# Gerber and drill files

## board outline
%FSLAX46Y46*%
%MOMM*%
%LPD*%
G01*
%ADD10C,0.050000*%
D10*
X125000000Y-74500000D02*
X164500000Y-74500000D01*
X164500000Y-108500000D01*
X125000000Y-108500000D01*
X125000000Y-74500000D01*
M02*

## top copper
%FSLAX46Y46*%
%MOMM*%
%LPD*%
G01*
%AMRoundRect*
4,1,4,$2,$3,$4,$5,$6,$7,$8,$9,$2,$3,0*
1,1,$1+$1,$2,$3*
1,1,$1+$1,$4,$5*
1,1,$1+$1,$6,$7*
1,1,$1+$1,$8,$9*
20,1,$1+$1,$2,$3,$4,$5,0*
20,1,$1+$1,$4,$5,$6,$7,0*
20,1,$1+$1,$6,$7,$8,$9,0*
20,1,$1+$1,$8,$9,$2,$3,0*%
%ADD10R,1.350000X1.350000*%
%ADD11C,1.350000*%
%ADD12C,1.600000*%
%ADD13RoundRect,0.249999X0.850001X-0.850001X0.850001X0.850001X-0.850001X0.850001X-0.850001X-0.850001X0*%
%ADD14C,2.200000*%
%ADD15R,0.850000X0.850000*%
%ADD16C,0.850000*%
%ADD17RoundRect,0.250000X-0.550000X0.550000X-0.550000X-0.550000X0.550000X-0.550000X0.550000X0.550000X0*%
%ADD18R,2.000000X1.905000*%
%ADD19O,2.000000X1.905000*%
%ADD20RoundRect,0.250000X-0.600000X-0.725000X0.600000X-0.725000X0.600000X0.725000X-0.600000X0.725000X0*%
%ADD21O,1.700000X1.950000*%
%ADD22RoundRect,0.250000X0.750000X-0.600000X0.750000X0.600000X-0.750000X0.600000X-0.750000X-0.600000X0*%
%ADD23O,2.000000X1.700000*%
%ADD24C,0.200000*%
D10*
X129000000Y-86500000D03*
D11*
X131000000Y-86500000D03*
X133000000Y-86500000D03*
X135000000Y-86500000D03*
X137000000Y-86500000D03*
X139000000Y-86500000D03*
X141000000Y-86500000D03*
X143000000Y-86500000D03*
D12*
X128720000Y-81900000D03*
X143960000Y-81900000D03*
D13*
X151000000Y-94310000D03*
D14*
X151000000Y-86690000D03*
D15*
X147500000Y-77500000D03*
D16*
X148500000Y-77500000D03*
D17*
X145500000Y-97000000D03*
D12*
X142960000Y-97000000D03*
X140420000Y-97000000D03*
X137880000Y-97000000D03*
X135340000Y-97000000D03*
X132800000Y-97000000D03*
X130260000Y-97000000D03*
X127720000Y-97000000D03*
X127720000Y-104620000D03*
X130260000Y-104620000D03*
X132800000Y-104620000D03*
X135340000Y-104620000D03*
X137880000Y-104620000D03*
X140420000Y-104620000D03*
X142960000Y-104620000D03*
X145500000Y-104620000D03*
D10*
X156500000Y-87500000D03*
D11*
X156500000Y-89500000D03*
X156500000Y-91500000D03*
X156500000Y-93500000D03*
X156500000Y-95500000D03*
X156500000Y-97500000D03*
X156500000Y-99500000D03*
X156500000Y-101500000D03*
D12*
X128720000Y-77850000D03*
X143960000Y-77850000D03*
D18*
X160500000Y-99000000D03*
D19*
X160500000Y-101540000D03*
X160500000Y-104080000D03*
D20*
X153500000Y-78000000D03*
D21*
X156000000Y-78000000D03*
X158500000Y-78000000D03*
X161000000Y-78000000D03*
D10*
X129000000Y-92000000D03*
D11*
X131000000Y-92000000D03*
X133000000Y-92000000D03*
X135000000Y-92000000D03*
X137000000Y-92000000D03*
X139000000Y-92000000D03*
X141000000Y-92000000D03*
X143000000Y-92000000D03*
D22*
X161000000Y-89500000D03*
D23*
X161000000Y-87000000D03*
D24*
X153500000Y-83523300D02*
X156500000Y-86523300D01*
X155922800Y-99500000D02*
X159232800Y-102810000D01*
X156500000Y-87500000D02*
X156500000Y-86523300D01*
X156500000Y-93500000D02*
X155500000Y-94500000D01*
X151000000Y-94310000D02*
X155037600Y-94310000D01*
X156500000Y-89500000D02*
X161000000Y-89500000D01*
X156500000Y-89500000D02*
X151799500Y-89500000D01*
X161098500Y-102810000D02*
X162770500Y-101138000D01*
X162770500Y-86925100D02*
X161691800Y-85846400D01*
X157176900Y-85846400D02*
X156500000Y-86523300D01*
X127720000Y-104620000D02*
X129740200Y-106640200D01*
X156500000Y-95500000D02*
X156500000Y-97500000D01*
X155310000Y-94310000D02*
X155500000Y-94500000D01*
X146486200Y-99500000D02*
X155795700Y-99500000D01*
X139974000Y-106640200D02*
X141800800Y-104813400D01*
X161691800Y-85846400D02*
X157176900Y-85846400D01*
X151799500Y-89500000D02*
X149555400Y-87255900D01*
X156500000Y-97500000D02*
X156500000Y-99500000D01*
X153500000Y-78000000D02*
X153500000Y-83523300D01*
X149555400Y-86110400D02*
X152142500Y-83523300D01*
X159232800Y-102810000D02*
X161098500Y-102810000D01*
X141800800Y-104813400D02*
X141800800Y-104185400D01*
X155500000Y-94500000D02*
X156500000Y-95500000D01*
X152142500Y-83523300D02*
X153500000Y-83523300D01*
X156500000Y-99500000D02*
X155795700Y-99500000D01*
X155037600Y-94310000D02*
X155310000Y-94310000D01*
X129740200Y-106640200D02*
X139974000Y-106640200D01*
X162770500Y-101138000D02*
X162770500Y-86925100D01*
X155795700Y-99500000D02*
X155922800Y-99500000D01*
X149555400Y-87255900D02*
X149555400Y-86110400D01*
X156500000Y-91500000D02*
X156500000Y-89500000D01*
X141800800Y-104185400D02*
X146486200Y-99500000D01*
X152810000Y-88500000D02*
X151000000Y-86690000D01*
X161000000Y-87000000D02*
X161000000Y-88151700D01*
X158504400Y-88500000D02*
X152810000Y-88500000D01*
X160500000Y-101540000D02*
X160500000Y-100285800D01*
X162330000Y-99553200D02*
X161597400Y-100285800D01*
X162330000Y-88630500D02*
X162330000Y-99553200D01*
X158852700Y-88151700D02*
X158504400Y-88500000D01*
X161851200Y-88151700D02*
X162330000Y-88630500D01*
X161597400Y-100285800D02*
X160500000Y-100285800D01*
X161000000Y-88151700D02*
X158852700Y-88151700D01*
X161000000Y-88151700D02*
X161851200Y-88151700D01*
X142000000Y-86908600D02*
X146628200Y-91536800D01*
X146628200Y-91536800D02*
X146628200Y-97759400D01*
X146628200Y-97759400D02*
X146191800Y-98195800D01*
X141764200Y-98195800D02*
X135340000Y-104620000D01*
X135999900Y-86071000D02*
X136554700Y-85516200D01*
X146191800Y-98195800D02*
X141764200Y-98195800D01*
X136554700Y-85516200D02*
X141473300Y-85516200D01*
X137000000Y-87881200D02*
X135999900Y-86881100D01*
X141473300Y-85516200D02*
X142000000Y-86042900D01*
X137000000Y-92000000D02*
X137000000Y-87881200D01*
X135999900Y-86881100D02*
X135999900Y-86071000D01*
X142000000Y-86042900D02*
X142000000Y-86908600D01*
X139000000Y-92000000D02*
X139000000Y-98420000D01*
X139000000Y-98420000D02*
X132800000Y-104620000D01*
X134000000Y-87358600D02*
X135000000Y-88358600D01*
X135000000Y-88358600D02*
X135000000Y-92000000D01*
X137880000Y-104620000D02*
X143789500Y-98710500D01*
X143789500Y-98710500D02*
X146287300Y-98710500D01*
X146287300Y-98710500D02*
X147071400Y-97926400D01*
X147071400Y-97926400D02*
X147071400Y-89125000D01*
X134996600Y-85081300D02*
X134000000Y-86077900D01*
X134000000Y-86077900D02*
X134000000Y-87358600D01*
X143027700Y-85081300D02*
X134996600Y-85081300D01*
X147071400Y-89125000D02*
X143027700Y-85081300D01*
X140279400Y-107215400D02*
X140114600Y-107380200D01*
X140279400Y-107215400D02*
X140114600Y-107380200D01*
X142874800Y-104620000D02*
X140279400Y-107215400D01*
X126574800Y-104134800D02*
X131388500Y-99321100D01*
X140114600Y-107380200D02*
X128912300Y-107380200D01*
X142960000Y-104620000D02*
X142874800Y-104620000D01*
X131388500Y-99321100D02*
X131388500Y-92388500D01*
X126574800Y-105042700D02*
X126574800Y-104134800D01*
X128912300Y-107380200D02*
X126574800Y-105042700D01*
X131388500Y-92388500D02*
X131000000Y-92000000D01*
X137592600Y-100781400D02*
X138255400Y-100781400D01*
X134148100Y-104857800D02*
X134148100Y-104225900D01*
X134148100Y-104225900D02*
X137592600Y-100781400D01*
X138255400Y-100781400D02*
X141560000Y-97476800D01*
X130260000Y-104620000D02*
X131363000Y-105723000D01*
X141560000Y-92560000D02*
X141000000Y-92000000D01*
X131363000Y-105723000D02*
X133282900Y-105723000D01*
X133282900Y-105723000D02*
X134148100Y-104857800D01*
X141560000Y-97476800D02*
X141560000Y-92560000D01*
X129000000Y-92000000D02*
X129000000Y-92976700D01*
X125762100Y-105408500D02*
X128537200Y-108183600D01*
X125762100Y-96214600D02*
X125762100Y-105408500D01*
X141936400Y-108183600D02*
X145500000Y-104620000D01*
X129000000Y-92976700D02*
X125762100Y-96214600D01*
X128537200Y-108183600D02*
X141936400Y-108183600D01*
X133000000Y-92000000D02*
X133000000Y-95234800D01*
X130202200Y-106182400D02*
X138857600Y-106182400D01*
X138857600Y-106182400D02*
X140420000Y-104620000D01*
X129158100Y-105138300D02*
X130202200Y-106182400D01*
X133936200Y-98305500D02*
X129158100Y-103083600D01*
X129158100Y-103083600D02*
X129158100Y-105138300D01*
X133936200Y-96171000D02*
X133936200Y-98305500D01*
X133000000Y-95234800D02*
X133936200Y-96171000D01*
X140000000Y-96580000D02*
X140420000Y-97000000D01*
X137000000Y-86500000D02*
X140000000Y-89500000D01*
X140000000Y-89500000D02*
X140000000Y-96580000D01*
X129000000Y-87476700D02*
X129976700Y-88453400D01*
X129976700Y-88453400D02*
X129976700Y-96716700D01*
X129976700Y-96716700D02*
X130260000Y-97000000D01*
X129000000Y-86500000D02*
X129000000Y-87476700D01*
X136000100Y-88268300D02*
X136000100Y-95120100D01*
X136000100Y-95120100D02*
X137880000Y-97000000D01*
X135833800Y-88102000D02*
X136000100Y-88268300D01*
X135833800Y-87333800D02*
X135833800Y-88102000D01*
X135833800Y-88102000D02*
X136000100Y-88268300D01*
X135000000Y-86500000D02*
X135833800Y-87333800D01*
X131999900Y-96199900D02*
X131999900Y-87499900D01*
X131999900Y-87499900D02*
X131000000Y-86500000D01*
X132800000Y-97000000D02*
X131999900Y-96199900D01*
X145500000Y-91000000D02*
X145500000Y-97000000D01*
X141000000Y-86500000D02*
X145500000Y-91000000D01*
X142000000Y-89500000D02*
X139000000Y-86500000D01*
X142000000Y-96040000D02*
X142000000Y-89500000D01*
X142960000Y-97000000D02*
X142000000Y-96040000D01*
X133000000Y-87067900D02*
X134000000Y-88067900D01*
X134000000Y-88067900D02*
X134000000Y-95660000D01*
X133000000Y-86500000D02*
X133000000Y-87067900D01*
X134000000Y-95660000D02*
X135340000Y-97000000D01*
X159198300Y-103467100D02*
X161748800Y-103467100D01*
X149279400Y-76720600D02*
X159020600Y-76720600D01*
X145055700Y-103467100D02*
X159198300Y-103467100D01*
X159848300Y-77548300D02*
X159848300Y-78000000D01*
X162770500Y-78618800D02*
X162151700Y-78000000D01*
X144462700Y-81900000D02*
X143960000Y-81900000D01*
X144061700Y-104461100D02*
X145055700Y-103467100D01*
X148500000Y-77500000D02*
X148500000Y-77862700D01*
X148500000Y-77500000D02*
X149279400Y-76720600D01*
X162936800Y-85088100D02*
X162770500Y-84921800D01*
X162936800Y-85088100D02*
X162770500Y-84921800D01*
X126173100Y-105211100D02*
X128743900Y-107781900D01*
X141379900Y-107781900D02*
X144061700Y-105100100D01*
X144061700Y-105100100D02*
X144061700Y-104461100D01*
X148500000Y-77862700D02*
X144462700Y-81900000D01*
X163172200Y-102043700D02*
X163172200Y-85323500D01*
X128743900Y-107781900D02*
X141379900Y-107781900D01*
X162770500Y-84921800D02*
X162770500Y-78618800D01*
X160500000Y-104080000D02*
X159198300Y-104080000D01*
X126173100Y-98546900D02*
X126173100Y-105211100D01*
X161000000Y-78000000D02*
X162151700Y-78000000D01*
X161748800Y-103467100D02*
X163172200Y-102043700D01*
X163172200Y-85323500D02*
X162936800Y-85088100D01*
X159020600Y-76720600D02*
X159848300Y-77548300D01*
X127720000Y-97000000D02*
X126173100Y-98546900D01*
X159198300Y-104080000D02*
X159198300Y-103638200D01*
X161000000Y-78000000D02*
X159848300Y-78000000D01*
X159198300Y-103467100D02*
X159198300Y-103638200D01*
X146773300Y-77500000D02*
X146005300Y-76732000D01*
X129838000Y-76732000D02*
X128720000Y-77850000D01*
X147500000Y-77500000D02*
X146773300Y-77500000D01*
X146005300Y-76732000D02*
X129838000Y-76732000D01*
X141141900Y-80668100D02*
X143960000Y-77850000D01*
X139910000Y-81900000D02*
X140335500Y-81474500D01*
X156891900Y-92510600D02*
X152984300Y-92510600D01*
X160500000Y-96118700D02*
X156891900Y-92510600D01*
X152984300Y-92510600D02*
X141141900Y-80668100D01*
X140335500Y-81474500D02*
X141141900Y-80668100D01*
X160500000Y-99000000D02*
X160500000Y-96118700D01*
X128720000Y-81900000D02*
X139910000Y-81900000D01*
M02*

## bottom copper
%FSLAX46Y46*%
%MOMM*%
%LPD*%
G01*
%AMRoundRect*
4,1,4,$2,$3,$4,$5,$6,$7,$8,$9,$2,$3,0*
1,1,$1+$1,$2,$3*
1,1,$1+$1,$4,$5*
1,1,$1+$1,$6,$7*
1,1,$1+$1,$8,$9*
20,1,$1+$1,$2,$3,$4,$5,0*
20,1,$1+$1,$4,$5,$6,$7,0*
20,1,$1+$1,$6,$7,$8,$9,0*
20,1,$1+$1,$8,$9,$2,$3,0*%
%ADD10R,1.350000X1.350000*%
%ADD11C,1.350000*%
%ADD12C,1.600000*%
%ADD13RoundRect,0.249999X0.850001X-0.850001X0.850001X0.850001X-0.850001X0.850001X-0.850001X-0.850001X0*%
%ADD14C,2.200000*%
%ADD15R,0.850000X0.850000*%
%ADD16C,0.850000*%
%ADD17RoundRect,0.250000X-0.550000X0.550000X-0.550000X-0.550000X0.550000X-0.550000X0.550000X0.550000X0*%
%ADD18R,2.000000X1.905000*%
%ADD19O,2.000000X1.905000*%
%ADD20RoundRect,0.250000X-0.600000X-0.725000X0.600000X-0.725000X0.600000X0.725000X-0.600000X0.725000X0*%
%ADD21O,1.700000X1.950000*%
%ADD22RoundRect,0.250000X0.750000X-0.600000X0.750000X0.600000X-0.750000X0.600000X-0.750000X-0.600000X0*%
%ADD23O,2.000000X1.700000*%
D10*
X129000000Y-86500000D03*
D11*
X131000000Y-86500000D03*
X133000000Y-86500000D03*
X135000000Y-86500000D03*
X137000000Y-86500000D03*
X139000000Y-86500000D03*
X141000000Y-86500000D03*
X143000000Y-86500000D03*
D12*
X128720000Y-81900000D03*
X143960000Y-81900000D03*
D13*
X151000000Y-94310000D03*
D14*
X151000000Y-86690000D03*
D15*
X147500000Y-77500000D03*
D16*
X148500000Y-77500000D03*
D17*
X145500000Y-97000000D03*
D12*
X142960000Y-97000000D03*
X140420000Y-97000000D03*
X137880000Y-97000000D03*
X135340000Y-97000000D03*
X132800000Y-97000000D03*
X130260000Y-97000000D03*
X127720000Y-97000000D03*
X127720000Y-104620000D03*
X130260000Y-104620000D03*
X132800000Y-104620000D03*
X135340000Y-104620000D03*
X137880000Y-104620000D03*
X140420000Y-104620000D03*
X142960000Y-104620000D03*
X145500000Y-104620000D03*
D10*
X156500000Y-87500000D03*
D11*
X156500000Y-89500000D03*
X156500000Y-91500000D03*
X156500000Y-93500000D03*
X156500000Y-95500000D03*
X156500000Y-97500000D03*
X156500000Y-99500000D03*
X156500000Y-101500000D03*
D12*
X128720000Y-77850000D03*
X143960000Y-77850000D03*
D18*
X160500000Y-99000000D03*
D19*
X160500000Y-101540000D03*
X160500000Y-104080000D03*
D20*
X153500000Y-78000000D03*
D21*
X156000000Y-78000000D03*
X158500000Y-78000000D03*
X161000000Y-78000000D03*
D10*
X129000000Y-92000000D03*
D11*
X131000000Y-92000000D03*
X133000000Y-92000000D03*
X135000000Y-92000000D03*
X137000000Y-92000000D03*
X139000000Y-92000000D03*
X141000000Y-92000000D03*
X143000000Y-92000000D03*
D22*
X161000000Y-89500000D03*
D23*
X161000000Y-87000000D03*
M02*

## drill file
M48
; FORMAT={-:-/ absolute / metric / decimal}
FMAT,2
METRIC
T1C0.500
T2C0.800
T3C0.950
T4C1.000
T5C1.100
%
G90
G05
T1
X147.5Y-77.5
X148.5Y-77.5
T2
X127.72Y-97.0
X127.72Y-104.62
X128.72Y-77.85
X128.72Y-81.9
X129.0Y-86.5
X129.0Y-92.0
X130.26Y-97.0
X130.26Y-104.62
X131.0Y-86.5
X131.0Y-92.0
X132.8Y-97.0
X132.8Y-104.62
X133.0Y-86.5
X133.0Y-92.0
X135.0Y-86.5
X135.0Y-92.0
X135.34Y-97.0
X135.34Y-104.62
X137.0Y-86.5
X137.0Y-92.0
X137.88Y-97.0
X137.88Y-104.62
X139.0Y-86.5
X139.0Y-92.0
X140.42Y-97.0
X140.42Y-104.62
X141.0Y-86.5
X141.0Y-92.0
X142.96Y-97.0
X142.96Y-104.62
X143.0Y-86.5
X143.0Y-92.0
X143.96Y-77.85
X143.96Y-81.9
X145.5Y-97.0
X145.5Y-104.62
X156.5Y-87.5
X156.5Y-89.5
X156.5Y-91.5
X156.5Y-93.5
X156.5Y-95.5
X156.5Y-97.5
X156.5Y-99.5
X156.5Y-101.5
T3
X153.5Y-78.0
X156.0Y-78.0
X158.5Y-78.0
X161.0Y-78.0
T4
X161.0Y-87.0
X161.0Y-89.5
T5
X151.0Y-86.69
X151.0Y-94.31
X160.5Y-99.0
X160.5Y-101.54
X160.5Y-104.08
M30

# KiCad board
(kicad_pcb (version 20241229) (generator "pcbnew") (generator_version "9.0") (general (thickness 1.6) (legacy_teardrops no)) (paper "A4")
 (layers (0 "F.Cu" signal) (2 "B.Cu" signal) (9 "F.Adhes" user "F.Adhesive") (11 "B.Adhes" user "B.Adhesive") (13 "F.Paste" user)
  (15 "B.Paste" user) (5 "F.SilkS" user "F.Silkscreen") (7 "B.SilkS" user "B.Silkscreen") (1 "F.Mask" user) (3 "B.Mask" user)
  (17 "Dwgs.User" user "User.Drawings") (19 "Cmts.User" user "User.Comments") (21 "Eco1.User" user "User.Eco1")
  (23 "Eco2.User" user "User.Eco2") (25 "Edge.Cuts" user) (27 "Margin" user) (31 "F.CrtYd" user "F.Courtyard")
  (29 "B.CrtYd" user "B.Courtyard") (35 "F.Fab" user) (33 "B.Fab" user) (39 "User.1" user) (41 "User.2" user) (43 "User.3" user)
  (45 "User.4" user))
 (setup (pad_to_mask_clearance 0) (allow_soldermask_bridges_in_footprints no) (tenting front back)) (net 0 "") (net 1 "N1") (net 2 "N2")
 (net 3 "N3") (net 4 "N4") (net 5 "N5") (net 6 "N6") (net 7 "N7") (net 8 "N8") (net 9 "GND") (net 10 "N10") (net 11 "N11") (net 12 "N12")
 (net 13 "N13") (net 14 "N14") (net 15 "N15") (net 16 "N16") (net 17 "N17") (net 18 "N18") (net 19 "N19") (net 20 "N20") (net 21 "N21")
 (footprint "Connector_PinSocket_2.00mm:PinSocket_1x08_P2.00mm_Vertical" (layer "F.Cu") (at 129 86.5 90)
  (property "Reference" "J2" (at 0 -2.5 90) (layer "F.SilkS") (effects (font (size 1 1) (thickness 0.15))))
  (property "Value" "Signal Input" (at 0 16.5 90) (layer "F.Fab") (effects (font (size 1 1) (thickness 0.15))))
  (pad "1" thru_hole rect (at 0 0 90) (size 1.35 1.35) (drill 0.8) (layers "*.Cu" "*.Mask") (remove_unused_layers no) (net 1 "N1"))
  (pad "2" thru_hole circle (at 0 2 90) (size 1.35 1.35) (drill 0.8) (layers "*.Cu" "*.Mask") (remove_unused_layers no) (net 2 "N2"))
  (pad "3" thru_hole circle (at 0 4 90) (size 1.35 1.35) (drill 0.8) (layers "*.Cu" "*.Mask") (remove_unused_layers no) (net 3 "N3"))
  (pad "4" thru_hole circle (at 0 6 90) (size 1.35 1.35) (drill 0.8) (layers "*.Cu" "*.Mask") (remove_unused_layers no) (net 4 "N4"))
  (pad "5" thru_hole circle (at 0 8 90) (size 1.35 1.35) (drill 0.8) (layers "*.Cu" "*.Mask") (remove_unused_layers no) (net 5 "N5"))
  (pad "6" thru_hole circle (at 0 10 90) (size 1.35 1.35) (drill 0.8) (layers "*.Cu" "*.Mask") (remove_unused_layers no) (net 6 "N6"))
  (pad "7" thru_hole circle (at 0 12 90) (size 1.35 1.35) (drill 0.8) (layers "*.Cu" "*.Mask") (remove_unused_layers no) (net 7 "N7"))
  (pad "8" thru_hole circle (at 0 14 90) (size 1.35 1.35) (drill 0.8) (layers "*.Cu" "*.Mask") (remove_unused_layers no)))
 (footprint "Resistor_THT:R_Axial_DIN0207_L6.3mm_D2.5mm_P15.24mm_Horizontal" (layer "F.Cu") (at 128.72 81.9)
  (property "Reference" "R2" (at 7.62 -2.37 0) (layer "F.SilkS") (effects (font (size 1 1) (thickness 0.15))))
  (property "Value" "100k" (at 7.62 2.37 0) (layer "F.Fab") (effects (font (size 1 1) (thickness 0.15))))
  (pad "1" thru_hole circle (at 0 0) (size 1.6 1.6) (drill 0.8) (layers "*.Cu" "*.Mask") (remove_unused_layers no) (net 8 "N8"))
  (pad "2" thru_hole circle (at 15.24 0) (size 1.6 1.6) (drill 0.8) (layers "*.Cu" "*.Mask") (remove_unused_layers no) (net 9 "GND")))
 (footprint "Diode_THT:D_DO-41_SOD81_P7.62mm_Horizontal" (layer "F.Cu") (at 151 94.31 90)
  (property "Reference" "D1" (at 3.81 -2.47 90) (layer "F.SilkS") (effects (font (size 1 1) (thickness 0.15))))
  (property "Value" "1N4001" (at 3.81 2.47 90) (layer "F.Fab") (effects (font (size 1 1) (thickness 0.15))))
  (pad "1" thru_hole roundrect (at 0 0 90) (size 2.2 2.2) (drill 1.1) (layers "*.Cu" "*.Mask") (remove_unused_layers no)
   (roundrect_rratio 0.113636) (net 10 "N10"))
  (pad "2" thru_hole circle (at 7.62 0 90) (size 2.2 2.2) (drill 1.1) (layers "*.Cu" "*.Mask") (remove_unused_layers no) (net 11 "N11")))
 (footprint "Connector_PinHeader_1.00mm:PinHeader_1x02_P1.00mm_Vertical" (layer "F.Cu") (at 147.5 77.5 90)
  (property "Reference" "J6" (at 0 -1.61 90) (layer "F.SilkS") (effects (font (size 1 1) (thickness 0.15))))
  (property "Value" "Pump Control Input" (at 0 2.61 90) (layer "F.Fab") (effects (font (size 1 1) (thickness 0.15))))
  (pad "1" thru_hole rect (at 0 0 90) (size 0.85 0.85) (drill 0.5) (layers "*.Cu" "*.Mask") (remove_unused_layers no) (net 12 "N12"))
  (pad "2" thru_hole circle (at 0 1 90) (size 0.85 0.85) (drill 0.5) (layers "*.Cu" "*.Mask") (remove_unused_layers no) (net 9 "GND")))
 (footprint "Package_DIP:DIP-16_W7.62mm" (layer "F.Cu") (at 145.5 97 -90)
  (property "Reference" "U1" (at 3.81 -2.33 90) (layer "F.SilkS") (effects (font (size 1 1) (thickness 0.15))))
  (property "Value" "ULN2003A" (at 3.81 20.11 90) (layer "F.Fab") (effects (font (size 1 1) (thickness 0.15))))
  (pad "1" thru_hole roundrect (at 0 0 270) (size 1.6 1.6) (drill 0.8) (layers "*.Cu" "*.Mask") (remove_unused_layers no)
   (roundrect_rratio 0.15625) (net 7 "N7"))
  (pad "2" thru_hole circle (at 0 2.54 270) (size 1.6 1.6) (drill 0.8) (layers "*.Cu" "*.Mask") (remove_unused_layers no) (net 6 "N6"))
  (pad "3" thru_hole circle (at 0 5.08 270) (size 1.6 1.6) (drill 0.8) (layers "*.Cu" "*.Mask") (remove_unused_layers no) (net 5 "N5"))
  (pad "4" thru_hole circle (at 0 7.62 270) (size 1.6 1.6) (drill 0.8) (layers "*.Cu" "*.Mask") (remove_unused_layers no) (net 4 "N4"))
  (pad "5" thru_hole circle (at 0 10.16 270) (size 1.6 1.6) (drill 0.8) (layers "*.Cu" "*.Mask") (remove_unused_layers no) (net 3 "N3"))
  (pad "6" thru_hole circle (at 0 12.7 270) (size 1.6 1.6) (drill 0.8) (layers "*.Cu" "*.Mask") (remove_unused_layers no) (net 2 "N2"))
  (pad "7" thru_hole circle (at 0 15.24 270) (size 1.6 1.6) (drill 0.8) (layers "*.Cu" "*.Mask") (remove_unused_layers no) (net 1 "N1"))
  (pad "8" thru_hole circle (at 0 17.78 270) (size 1.6 1.6) (drill 0.8) (layers "*.Cu" "*.Mask") (remove_unused_layers no) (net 9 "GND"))
  (pad "9" thru_hole circle (at 7.62 17.78 270) (size 1.6 1.6) (drill 0.8) (layers "*.Cu" "*.Mask") (remove_unused_layers no) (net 10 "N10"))
  (pad "10" thru_hole circle (at 7.62 15.24 270) (size 1.6 1.6) (drill 0.8) (layers "*.Cu" "*.Mask") (remove_unused_layers no)
   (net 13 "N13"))
  (pad "11" thru_hole circle (at 7.62 12.7 270) (size 1.6 1.6) (drill 0.8) (layers "*.Cu" "*.Mask") (remove_unused_layers no) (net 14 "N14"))
  (pad "12" thru_hole circle (at 7.62 10.16 270) (size 1.6 1.6) (drill 0.8) (layers "*.Cu" "*.Mask") (remove_unused_layers no)
   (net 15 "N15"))
  (pad "13" thru_hole circle (at 7.62 7.62 270) (size 1.6 1.6) (drill 0.8) (layers "*.Cu" "*.Mask") (remove_unused_layers no) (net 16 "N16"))
  (pad "14" thru_hole circle (at 7.62 5.08 270) (size 1.6 1.6) (drill 0.8) (layers "*.Cu" "*.Mask") (remove_unused_layers no) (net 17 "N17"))
  (pad "15" thru_hole circle (at 7.62 2.54 270) (size 1.6 1.6) (drill 0.8) (layers "*.Cu" "*.Mask") (remove_unused_layers no) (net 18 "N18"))
  (pad "16" thru_hole circle (at 7.62 0 270) (size 1.6 1.6) (drill 0.8) (layers "*.Cu" "*.Mask") (remove_unused_layers no) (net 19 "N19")))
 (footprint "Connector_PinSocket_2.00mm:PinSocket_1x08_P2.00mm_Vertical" (layer "F.Cu") (at 156.5 87.5)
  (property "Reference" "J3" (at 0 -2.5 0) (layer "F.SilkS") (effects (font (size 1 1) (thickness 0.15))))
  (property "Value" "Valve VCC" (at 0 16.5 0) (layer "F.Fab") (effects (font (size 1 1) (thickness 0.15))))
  (pad "1" thru_hole rect (at 0 0) (size 1.35 1.35) (drill 0.8) (layers "*.Cu" "*.Mask") (remove_unused_layers no) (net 10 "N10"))
  (pad "2" thru_hole circle (at 0 2) (size 1.35 1.35) (drill 0.8) (layers "*.Cu" "*.Mask") (remove_unused_layers no) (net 10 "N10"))
  (pad "3" thru_hole circle (at 0 4) (size 1.35 1.35) (drill 0.8) (layers "*.Cu" "*.Mask") (remove_unused_layers no) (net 10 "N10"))
  (pad "4" thru_hole circle (at 0 6) (size 1.35 1.35) (drill 0.8) (layers "*.Cu" "*.Mask") (remove_unused_layers no) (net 10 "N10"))
  (pad "5" thru_hole circle (at 0 8) (size 1.35 1.35) (drill 0.8) (layers "*.Cu" "*.Mask") (remove_unused_layers no) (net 10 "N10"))
  (pad "6" thru_hole circle (at 0 10) (size 1.35 1.35) (drill 0.8) (layers "*.Cu" "*.Mask") (remove_unused_layers no) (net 10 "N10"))
  (pad "7" thru_hole circle (at 0 12) (size 1.35 1.35) (drill 0.8) (layers "*.Cu" "*.Mask") (remove_unused_layers no) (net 10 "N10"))
  (pad "8" thru_hole circle (at 0 14) (size 1.35 1.35) (drill 0.8) (layers "*.Cu" "*.Mask") (remove_unused_layers no)))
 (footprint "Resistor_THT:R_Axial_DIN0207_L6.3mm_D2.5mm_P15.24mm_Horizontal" (layer "F.Cu") (at 128.72 77.85)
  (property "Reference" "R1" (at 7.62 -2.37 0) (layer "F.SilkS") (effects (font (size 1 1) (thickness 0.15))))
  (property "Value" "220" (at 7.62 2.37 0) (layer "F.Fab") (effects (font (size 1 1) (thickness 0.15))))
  (pad "1" thru_hole circle (at 0 0) (size 1.6 1.6) (drill 0.8) (layers "*.Cu" "*.Mask") (remove_unused_layers no) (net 12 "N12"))
  (pad "2" thru_hole circle (at 15.24 0) (size 1.6 1.6) (drill 0.8) (layers "*.Cu" "*.Mask") (remove_unused_layers no) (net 8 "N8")))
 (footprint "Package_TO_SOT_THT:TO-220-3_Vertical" (layer "F.Cu") (at 160.5 99 -90)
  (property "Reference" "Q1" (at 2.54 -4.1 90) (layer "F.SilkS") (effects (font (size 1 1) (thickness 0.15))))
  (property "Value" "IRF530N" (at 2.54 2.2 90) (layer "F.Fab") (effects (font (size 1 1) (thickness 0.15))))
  (pad "1" thru_hole rect (at 0 0 270) (size 1.905 2) (drill 1.1) (layers "*.Cu" "*.Mask") (remove_unused_layers no) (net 8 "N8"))
  (pad "2" thru_hole oval (at 2.54 0 270) (size 1.905 2) (drill 1.1) (layers "*.Cu" "*.Mask") (remove_unused_layers no) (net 11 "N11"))
  (pad "3" thru_hole oval (at 5.08 0 270) (size 1.905 2) (drill 1.1) (layers "*.Cu" "*.Mask") (remove_unused_layers no) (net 9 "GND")))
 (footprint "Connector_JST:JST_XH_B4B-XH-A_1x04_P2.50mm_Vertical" (layer "F.Cu") (at 153.5 78)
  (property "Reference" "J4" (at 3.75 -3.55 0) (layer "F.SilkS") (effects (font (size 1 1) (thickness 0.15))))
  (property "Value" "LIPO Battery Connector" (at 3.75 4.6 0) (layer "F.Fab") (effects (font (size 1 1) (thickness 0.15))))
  (pad "1" thru_hole roundrect (at 0 0) (size 1.7 1.95) (drill 0.95) (layers "*.Cu" "*.Mask") (remove_unused_layers no)
   (roundrect_rratio 0.147059) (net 10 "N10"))
  (pad "2" thru_hole oval (at 2.5 0) (size 1.7 1.95) (drill 0.95) (layers "*.Cu" "*.Mask") (remove_unused_layers no) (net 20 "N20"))
  (pad "3" thru_hole oval (at 5 0) (size 1.7 1.95) (drill 0.95) (layers "*.Cu" "*.Mask") (remove_unused_layers no) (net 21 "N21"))
  (pad "4" thru_hole oval (at 7.5 0) (size 1.7 1.95) (drill 0.95) (layers "*.Cu" "*.Mask") (remove_unused_layers no) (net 9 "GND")))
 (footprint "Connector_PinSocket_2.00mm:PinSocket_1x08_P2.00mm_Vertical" (layer "F.Cu") (at 129 92 90)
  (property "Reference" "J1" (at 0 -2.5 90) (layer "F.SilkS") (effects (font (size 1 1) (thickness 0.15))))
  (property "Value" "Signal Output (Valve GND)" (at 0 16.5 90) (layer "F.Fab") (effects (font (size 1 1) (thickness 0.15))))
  (pad "1" thru_hole rect (at 0 0 90) (size 1.35 1.35) (drill 0.8) (layers "*.Cu" "*.Mask") (remove_unused_layers no) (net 19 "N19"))
  (pad "2" thru_hole circle (at 0 2 90) (size 1.35 1.35) (drill 0.8) (layers "*.Cu" "*.Mask") (remove_unused_layers no) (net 18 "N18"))
  (pad "3" thru_hole circle (at 0 4 90) (size 1.35 1.35) (drill 0.8) (layers "*.Cu" "*.Mask") (remove_unused_layers no) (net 17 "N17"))
  (pad "4" thru_hole circle (at 0 6 90) (size 1.35 1.35) (drill 0.8) (layers "*.Cu" "*.Mask") (remove_unused_layers no) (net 16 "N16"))
  (pad "5" thru_hole circle (at 0 8 90) (size 1.35 1.35) (drill 0.8) (layers "*.Cu" "*.Mask") (remove_unused_layers no) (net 15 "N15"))
  (pad "6" thru_hole circle (at 0 10 90) (size 1.35 1.35) (drill 0.8) (layers "*.Cu" "*.Mask") (remove_unused_layers no) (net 14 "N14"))
  (pad "7" thru_hole circle (at 0 12 90) (size 1.35 1.35) (drill 0.8) (layers "*.Cu" "*.Mask") (remove_unused_layers no) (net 13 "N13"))
  (pad "8" thru_hole circle (at 0 14 90) (size 1.35 1.35) (drill 0.8) (layers "*.Cu" "*.Mask") (remove_unused_layers no)))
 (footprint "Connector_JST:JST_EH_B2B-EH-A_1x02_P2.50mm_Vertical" (layer "F.Cu") (at 161 89.5 90)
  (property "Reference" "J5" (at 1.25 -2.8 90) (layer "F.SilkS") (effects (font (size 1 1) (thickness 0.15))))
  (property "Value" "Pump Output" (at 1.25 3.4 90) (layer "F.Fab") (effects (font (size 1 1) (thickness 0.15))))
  (pad "1" thru_hole roundrect (at 0 0 90) (size 1.7 2) (drill 1) (layers "*.Cu" "*.Mask") (remove_unused_layers no)
   (roundrect_rratio 0.147059) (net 10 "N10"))
  (pad "2" thru_hole oval (at 2.5 0 90) (size 1.7 2) (drill 1) (layers "*.Cu" "*.Mask") (remove_unused_layers no) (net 11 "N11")))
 (gr_rect (start 125 74.5) (end 164.5 108.5) (stroke (width 0.05) (type default)) (fill no) (layer "Edge.Cuts"))
 (segment (start 153.5 83.5233) (end 156.5 86.5233) (width 0.2) (layer "F.Cu") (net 10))
 (segment (start 155.9228 99.5) (end 159.2328 102.81) (width 0.2) (layer "F.Cu") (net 10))
 (segment (start 156.5 87.5) (end 156.5 86.5233) (width 0.2) (layer "F.Cu") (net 10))
 (segment (start 156.5 93.5) (end 155.5 94.5) (width 0.2) (layer "F.Cu") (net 10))
 (segment (start 151 94.31) (end 155.0376 94.31) (width 0.2) (layer "F.Cu") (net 10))
 (segment (start 156.5 89.5) (end 161 89.5) (width 0.2) (layer "F.Cu") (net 10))
 (segment (start 156.5 89.5) (end 151.7995 89.5) (width 0.2) (layer "F.Cu") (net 10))
 (segment (start 161.0985 102.81) (end 162.7705 101.138) (width 0.2) (layer "F.Cu") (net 10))
 (segment (start 162.7705 86.9251) (end 161.6918 85.8464) (width 0.2) (layer "F.Cu") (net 10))
 (segment (start 157.1769 85.8464) (end 156.5 86.5233) (width 0.2) (layer "F.Cu") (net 10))
 (segment (start 127.72 104.62) (end 129.7402 106.6402) (width 0.2) (layer "F.Cu") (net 10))
 (segment (start 156.5 95.5) (end 156.5 97.5) (width 0.2) (layer "F.Cu") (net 10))
 (segment (start 155.31 94.31) (end 155.5 94.5) (width 0.2) (layer "F.Cu") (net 10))
 (segment (start 146.4862 99.5) (end 155.7957 99.5) (width 0.2) (layer "F.Cu") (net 10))
 (segment (start 139.974 106.6402) (end 141.8008 104.8134) (width 0.2) (layer "F.Cu") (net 10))
 (segment (start 161.6918 85.8464) (end 157.1769 85.8464) (width 0.2) (layer "F.Cu") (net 10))
 (segment (start 151.7995 89.5) (end 149.5554 87.2559) (width 0.2) (layer "F.Cu") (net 10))
 (segment (start 156.5 97.5) (end 156.5 99.5) (width 0.2) (layer "F.Cu") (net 10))
 (segment (start 153.5 78) (end 153.5 83.5233) (width 0.2) (layer "F.Cu") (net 10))
 (segment (start 149.5554 86.1104) (end 152.1425 83.5233) (width 0.2) (layer "F.Cu") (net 10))
 (segment (start 159.2328 102.81) (end 161.0985 102.81) (width 0.2) (layer "F.Cu") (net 10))
 (segment (start 141.8008 104.8134) (end 141.8008 104.1854) (width 0.2) (layer "F.Cu") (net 10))
 (segment (start 155.5 94.5) (end 156.5 95.5) (width 0.2) (layer "F.Cu") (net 10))
 (segment (start 152.1425 83.5233) (end 153.5 83.5233) (width 0.2) (layer "F.Cu") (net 10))
 (segment (start 156.5 99.5) (end 155.7957 99.5) (width 0.2) (layer "F.Cu") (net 10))
 (segment (start 155.0376 94.31) (end 155.31 94.31) (width 0.2) (layer "F.Cu") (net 10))
 (segment (start 129.7402 106.6402) (end 139.974 106.6402) (width 0.2) (layer "F.Cu") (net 10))
 (segment (start 162.7705 101.138) (end 162.7705 86.9251) (width 0.2) (layer "F.Cu") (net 10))
 (segment (start 155.7957 99.5) (end 155.9228 99.5) (width 0.2) (layer "F.Cu") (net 10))
 (segment (start 149.5554 87.2559) (end 149.5554 86.1104) (width 0.2) (layer "F.Cu") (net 10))
 (segment (start 156.5 91.5) (end 156.5 89.5) (width 0.2) (layer "F.Cu") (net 10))
 (segment (start 141.8008 104.1854) (end 146.4862 99.5) (width 0.2) (layer "F.Cu") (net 10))
 (segment (start 152.81 88.5) (end 151 86.69) (width 0.2) (layer "F.Cu") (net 11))
 (segment (start 161 87) (end 161 88.1517) (width 0.2) (layer "F.Cu") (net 11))
 (segment (start 158.5044 88.5) (end 152.81 88.5) (width 0.2) (layer "F.Cu") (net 11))
 (segment (start 160.5 101.54) (end 160.5 100.2858) (width 0.2) (layer "F.Cu") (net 11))
 (segment (start 162.33 99.5532) (end 161.5974 100.2858) (width 0.2) (layer "F.Cu") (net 11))
 (segment (start 162.33 88.6305) (end 162.33 99.5532) (width 0.2) (layer "F.Cu") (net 11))
 (segment (start 158.8527 88.1517) (end 158.5044 88.5) (width 0.2) (layer "F.Cu") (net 11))
 (segment (start 161.8512 88.1517) (end 162.33 88.6305) (width 0.2) (layer "F.Cu") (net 11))
 (segment (start 161.5974 100.2858) (end 160.5 100.2858) (width 0.2) (layer "F.Cu") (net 11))
 (segment (start 161 88.1517) (end 158.8527 88.1517) (width 0.2) (layer "F.Cu") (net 11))
 (segment (start 161 88.1517) (end 161.8512 88.1517) (width 0.2) (layer "F.Cu") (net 11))
 (segment (start 142 86.9086) (end 146.6282 91.5368) (width 0.2) (layer "F.Cu") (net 15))
 (segment (start 146.6282 91.5368) (end 146.6282 97.7594) (width 0.2) (layer "F.Cu") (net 15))
 (segment (start 146.6282 97.7594) (end 146.1918 98.1958) (width 0.2) (layer "F.Cu") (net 15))
 (segment (start 141.7642 98.1958) (end 135.34 104.62) (width 0.2) (layer "F.Cu") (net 15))
 (segment (start 135.9999 86.071) (end 136.5547 85.5162) (width 0.2) (layer "F.Cu") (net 15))
 (segment (start 146.1918 98.1958) (end 141.7642 98.1958) (width 0.2) (layer "F.Cu") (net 15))
 (segment (start 136.5547 85.5162) (end 141.4733 85.5162) (width 0.2) (layer "F.Cu") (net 15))
 (segment (start 137 87.8812) (end 135.9999 86.8811) (width 0.2) (layer "F.Cu") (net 15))
 (segment (start 141.4733 85.5162) (end 142 86.0429) (width 0.2) (layer "F.Cu") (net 15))
 (segment (start 137 92) (end 137 87.8812) (width 0.2) (layer "F.Cu") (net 15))
 (segment (start 135.9999 86.8811) (end 135.9999 86.071) (width 0.2) (layer "F.Cu") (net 15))
 (segment (start 142 86.0429) (end 142 86.9086) (width 0.2) (layer "F.Cu") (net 15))
 (segment (start 139 92) (end 139 98.42) (width 0.2) (layer "F.Cu") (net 14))
 (segment (start 139 98.42) (end 132.8 104.62) (width 0.2) (layer "F.Cu") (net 14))
 (segment (start 134 87.3586) (end 135 88.3586) (width 0.2) (layer "F.Cu") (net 16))
 (segment (start 135 88.3586) (end 135 92) (width 0.2) (layer "F.Cu") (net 16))
 (segment (start 137.88 104.62) (end 143.7895 98.7105) (width 0.2) (layer "F.Cu") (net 16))
 (segment (start 143.7895 98.7105) (end 146.2873 98.7105) (width 0.2) (layer "F.Cu") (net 16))
 (segment (start 146.2873 98.7105) (end 147.0714 97.9264) (width 0.2) (layer "F.Cu") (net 16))
 (segment (start 147.0714 97.9264) (end 147.0714 89.125) (width 0.2) (layer "F.Cu") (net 16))
 (segment (start 134.9966 85.0813) (end 134 86.0779) (width 0.2) (layer "F.Cu") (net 16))
 (segment (start 134 86.0779) (end 134 87.3586) (width 0.2) (layer "F.Cu") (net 16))
 (segment (start 143.0277 85.0813) (end 134.9966 85.0813) (width 0.2) (layer "F.Cu") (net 16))
 (segment (start 147.0714 89.125) (end 143.0277 85.0813) (width 0.2) (layer "F.Cu") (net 16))
 (segment (start 140.2794 107.2154) (end 140.1146 107.3802) (width 0.2) (layer "F.Cu") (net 18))
 (segment (start 140.2794 107.2154) (end 140.1146 107.3802) (width 0.2) (layer "F.Cu") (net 18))
 (segment (start 142.8748 104.62) (end 140.2794 107.2154) (width 0.2) (layer "F.Cu") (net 18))
 (segment (start 126.5748 104.1348) (end 131.3885 99.3211) (width 0.2) (layer "F.Cu") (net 18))
 (segment (start 140.1146 107.3802) (end 128.9123 107.3802) (width 0.2) (layer "F.Cu") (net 18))
 (segment (start 142.96 104.62) (end 142.8748 104.62) (width 0.2) (layer "F.Cu") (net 18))
 (segment (start 131.3885 99.3211) (end 131.3885 92.3885) (width 0.2) (layer "F.Cu") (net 18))
 (segment (start 126.5748 105.0427) (end 126.5748 104.1348) (width 0.2) (layer "F.Cu") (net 18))
 (segment (start 128.9123 107.3802) (end 126.5748 105.0427) (width 0.2) (layer "F.Cu") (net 18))
 (segment (start 131.3885 92.3885) (end 131 92) (width 0.2) (layer "F.Cu") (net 18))
 (segment (start 137.5926 100.7814) (end 138.2554 100.7814) (width 0.2) (layer "F.Cu") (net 13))
 (segment (start 134.1481 104.8578) (end 134.1481 104.2259) (width 0.2) (layer "F.Cu") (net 13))
 (segment (start 134.1481 104.2259) (end 137.5926 100.7814) (width 0.2) (layer "F.Cu") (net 13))
 (segment (start 138.2554 100.7814) (end 141.56 97.4768) (width 0.2) (layer "F.Cu") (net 13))
 (segment (start 130.26 104.62) (end 131.363 105.723) (width 0.2) (layer "F.Cu") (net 13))
 (segment (start 141.56 92.56) (end 141 92) (width 0.2) (layer "F.Cu") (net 13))
 (segment (start 131.363 105.723) (end 133.2829 105.723) (width 0.2) (layer "F.Cu") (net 13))
 (segment (start 133.2829 105.723) (end 134.1481 104.8578) (width 0.2) (layer "F.Cu") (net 13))
 (segment (start 141.56 97.4768) (end 141.56 92.56) (width 0.2) (layer "F.Cu") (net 13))
 (segment (start 129 92) (end 129 92.9767) (width 0.2) (layer "F.Cu") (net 19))
 (segment (start 125.7621 105.4085) (end 128.5372 108.1836) (width 0.2) (layer "F.Cu") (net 19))
 (segment (start 125.7621 96.2146) (end 125.7621 105.4085) (width 0.2) (layer "F.Cu") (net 19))
 (segment (start 141.9364 108.1836) (end 145.5 104.62) (width 0.2) (layer "F.Cu") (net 19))
 (segment (start 129 92.9767) (end 125.7621 96.2146) (width 0.2) (layer "F.Cu") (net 19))
 (segment (start 128.5372 108.1836) (end 141.9364 108.1836) (width 0.2) (layer "F.Cu") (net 19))
 (segment (start 133 92) (end 133 95.2348) (width 0.2) (layer "F.Cu") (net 17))
 (segment (start 130.2022 106.1824) (end 138.8576 106.1824) (width 0.2) (layer "F.Cu") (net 17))
 (segment (start 138.8576 106.1824) (end 140.42 104.62) (width 0.2) (layer "F.Cu") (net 17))
 (segment (start 129.1581 105.1383) (end 130.2022 106.1824) (width 0.2) (layer "F.Cu") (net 17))
 (segment (start 133.9362 98.3055) (end 129.1581 103.0836) (width 0.2) (layer "F.Cu") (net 17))
 (segment (start 129.1581 103.0836) (end 129.1581 105.1383) (width 0.2) (layer "F.Cu") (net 17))
 (segment (start 133.9362 96.171) (end 133.9362 98.3055) (width 0.2) (layer "F.Cu") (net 17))
 (segment (start 133 95.2348) (end 133.9362 96.171) (width 0.2) (layer "F.Cu") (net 17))
 (segment (start 140 96.58) (end 140.42 97) (width 0.2) (layer "F.Cu") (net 5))
 (segment (start 137 86.5) (end 140 89.5) (width 0.2) (layer "F.Cu") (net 5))
 (segment (start 140 89.5) (end 140 96.58) (width 0.2) (layer "F.Cu") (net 5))
 (segment (start 129 87.4767) (end 129.9767 88.4534) (width 0.2) (layer "F.Cu") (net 1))
 (segment (start 129.9767 88.4534) (end 129.9767 96.7167) (width 0.2) (layer "F.Cu") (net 1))
 (segment (start 129.9767 96.7167) (end 130.26 97) (width 0.2) (layer "F.Cu") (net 1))
 (segment (start 129 86.5) (end 129 87.4767) (width 0.2) (layer "F.Cu") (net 1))
 (segment (start 136.0001 88.2683) (end 136.0001 95.1201) (width 0.2) (layer "F.Cu") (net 4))
 (segment (start 136.0001 95.1201) (end 137.88 97) (width 0.2) (layer "F.Cu") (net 4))
 (segment (start 135.8338 88.102) (end 136.0001 88.2683) (width 0.2) (layer "F.Cu") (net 4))
 (segment (start 135.8338 87.3338) (end 135.8338 88.102) (width 0.2) (layer "F.Cu") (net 4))
 (segment (start 135.8338 88.102) (end 136.0001 88.2683) (width 0.2) (layer "F.Cu") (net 4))
 (segment (start 135 86.5) (end 135.8338 87.3338) (width 0.2) (layer "F.Cu") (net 4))
 (segment (start 131.9999 96.1999) (end 131.9999 87.4999) (width 0.2) (layer "F.Cu") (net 2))
 (segment (start 131.9999 87.4999) (end 131 86.5) (width 0.2) (layer "F.Cu") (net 2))
 (segment (start 132.8 97) (end 131.9999 96.1999) (width 0.2) (layer "F.Cu") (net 2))
 (segment (start 145.5 91) (end 145.5 97) (width 0.2) (layer "F.Cu") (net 7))
 (segment (start 141 86.5) (end 145.5 91) (width 0.2) (layer "F.Cu") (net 7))
 (segment (start 142 89.5) (end 139 86.5) (width 0.2) (layer "F.Cu") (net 6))
 (segment (start 142 96.04) (end 142 89.5) (width 0.2) (layer "F.Cu") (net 6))
 (segment (start 142.96 97) (end 142 96.04) (width 0.2) (layer "F.Cu") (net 6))
 (segment (start 133 87.0679) (end 134 88.0679) (width 0.2) (layer "F.Cu") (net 3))
 (segment (start 134 88.0679) (end 134 95.66) (width 0.2) (layer "F.Cu") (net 3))
 (segment (start 133 86.5) (end 133 87.0679) (width 0.2) (layer "F.Cu") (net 3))
 (segment (start 134 95.66) (end 135.34 97) (width 0.2) (layer "F.Cu") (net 3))
 (segment (start 159.1983 103.4671) (end 161.7488 103.4671) (width 0.2) (layer "F.Cu") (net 9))
 (segment (start 149.2794 76.7206) (end 159.0206 76.7206) (width 0.2) (layer "F.Cu") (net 9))
 (segment (start 145.0557 103.4671) (end 159.1983 103.4671) (width 0.2) (layer "F.Cu") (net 9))
 (segment (start 159.8483 77.5483) (end 159.8483 78) (width 0.2) (layer "F.Cu") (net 9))
 (segment (start 162.7705 78.6188) (end 162.1517 78) (width 0.2) (layer "F.Cu") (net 9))
 (segment (start 144.4627 81.9) (end 143.96 81.9) (width 0.2) (layer "F.Cu") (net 9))
 (segment (start 144.0617 104.4611) (end 145.0557 103.4671) (width 0.2) (layer "F.Cu") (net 9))
 (segment (start 148.5 77.5) (end 148.5 77.8627) (width 0.2) (layer "F.Cu") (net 9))
 (segment (start 148.5 77.5) (end 149.2794 76.7206) (width 0.2) (layer "F.Cu") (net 9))
 (segment (start 162.9368 85.0881) (end 162.7705 84.9218) (width 0.2) (layer "F.Cu") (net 9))
 (segment (start 162.9368 85.0881) (end 162.7705 84.9218) (width 0.2) (layer "F.Cu") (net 9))
 (segment (start 126.1731 105.2111) (end 128.7439 107.7819) (width 0.2) (layer "F.Cu") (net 9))
 (segment (start 141.3799 107.7819) (end 144.0617 105.1001) (width 0.2) (layer "F.Cu") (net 9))
 (segment (start 144.0617 105.1001) (end 144.0617 104.4611) (width 0.2) (layer "F.Cu") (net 9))
 (segment (start 148.5 77.8627) (end 144.4627 81.9) (width 0.2) (layer "F.Cu") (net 9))
 (segment (start 163.1722 102.0437) (end 163.1722 85.3235) (width 0.2) (layer "F.Cu") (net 9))
 (segment (start 128.7439 107.7819) (end 141.3799 107.7819) (width 0.2) (layer "F.Cu") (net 9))
 (segment (start 162.7705 84.9218) (end 162.7705 78.6188) (width 0.2) (layer "F.Cu") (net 9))
 (segment (start 160.5 104.08) (end 159.1983 104.08) (width 0.2) (layer "F.Cu") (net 9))
 (segment (start 126.1731 98.5469) (end 126.1731 105.2111) (width 0.2) (layer "F.Cu") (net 9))
 (segment (start 161 78) (end 162.1517 78) (width 0.2) (layer "F.Cu") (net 9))
 (segment (start 161.7488 103.4671) (end 163.1722 102.0437) (width 0.2) (layer "F.Cu") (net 9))
 (segment (start 163.1722 85.3235) (end 162.9368 85.0881) (width 0.2) (layer "F.Cu") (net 9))
 (segment (start 159.0206 76.7206) (end 159.8483 77.5483) (width 0.2) (layer "F.Cu") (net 9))
 (segment (start 127.72 97) (end 126.1731 98.5469) (width 0.2) (layer "F.Cu") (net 9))
 (segment (start 159.1983 104.08) (end 159.1983 103.6382) (width 0.2) (layer "F.Cu") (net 9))
 (segment (start 161 78) (end 159.8483 78) (width 0.2) (layer "F.Cu") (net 9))
 (segment (start 159.1983 103.4671) (end 159.1983 103.6382) (width 0.2) (layer "F.Cu") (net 9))
 (segment (start 146.7733 77.5) (end 146.0053 76.732) (width 0.2) (layer "F.Cu") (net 12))
 (segment (start 129.838 76.732) (end 128.72 77.85) (width 0.2) (layer "F.Cu") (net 12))
 (segment (start 147.5 77.5) (end 146.7733 77.5) (width 0.2) (layer "F.Cu") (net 12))
 (segment (start 146.0053 76.732) (end 129.838 76.732) (width 0.2) (layer "F.Cu") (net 12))
 (segment (start 141.1419 80.6681) (end 143.96 77.85) (width 0.2) (layer "F.Cu") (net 8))
 (segment (start 139.91 81.9) (end 140.3355 81.4745) (width 0.2) (layer "F.Cu") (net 8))
 (segment (start 156.8919 92.5106) (end 152.9843 92.5106) (width 0.2) (layer "F.Cu") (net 8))
 (segment (start 160.5 96.1187) (end 156.8919 92.5106) (width 0.2) (layer "F.Cu") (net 8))
 (segment (start 152.9843 92.5106) (end 141.1419 80.6681) (width 0.2) (layer "F.Cu") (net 8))
 (segment (start 140.3355 81.4745) (end 141.1419 80.6681) (width 0.2) (layer "F.Cu") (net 8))
 (segment (start 160.5 99) (end 160.5 96.1187) (width 0.2) (layer "F.Cu") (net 8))
 (segment (start 128.72 81.9) (end 139.91 81.9) (width 0.2) (layer "F.Cu") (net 8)))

